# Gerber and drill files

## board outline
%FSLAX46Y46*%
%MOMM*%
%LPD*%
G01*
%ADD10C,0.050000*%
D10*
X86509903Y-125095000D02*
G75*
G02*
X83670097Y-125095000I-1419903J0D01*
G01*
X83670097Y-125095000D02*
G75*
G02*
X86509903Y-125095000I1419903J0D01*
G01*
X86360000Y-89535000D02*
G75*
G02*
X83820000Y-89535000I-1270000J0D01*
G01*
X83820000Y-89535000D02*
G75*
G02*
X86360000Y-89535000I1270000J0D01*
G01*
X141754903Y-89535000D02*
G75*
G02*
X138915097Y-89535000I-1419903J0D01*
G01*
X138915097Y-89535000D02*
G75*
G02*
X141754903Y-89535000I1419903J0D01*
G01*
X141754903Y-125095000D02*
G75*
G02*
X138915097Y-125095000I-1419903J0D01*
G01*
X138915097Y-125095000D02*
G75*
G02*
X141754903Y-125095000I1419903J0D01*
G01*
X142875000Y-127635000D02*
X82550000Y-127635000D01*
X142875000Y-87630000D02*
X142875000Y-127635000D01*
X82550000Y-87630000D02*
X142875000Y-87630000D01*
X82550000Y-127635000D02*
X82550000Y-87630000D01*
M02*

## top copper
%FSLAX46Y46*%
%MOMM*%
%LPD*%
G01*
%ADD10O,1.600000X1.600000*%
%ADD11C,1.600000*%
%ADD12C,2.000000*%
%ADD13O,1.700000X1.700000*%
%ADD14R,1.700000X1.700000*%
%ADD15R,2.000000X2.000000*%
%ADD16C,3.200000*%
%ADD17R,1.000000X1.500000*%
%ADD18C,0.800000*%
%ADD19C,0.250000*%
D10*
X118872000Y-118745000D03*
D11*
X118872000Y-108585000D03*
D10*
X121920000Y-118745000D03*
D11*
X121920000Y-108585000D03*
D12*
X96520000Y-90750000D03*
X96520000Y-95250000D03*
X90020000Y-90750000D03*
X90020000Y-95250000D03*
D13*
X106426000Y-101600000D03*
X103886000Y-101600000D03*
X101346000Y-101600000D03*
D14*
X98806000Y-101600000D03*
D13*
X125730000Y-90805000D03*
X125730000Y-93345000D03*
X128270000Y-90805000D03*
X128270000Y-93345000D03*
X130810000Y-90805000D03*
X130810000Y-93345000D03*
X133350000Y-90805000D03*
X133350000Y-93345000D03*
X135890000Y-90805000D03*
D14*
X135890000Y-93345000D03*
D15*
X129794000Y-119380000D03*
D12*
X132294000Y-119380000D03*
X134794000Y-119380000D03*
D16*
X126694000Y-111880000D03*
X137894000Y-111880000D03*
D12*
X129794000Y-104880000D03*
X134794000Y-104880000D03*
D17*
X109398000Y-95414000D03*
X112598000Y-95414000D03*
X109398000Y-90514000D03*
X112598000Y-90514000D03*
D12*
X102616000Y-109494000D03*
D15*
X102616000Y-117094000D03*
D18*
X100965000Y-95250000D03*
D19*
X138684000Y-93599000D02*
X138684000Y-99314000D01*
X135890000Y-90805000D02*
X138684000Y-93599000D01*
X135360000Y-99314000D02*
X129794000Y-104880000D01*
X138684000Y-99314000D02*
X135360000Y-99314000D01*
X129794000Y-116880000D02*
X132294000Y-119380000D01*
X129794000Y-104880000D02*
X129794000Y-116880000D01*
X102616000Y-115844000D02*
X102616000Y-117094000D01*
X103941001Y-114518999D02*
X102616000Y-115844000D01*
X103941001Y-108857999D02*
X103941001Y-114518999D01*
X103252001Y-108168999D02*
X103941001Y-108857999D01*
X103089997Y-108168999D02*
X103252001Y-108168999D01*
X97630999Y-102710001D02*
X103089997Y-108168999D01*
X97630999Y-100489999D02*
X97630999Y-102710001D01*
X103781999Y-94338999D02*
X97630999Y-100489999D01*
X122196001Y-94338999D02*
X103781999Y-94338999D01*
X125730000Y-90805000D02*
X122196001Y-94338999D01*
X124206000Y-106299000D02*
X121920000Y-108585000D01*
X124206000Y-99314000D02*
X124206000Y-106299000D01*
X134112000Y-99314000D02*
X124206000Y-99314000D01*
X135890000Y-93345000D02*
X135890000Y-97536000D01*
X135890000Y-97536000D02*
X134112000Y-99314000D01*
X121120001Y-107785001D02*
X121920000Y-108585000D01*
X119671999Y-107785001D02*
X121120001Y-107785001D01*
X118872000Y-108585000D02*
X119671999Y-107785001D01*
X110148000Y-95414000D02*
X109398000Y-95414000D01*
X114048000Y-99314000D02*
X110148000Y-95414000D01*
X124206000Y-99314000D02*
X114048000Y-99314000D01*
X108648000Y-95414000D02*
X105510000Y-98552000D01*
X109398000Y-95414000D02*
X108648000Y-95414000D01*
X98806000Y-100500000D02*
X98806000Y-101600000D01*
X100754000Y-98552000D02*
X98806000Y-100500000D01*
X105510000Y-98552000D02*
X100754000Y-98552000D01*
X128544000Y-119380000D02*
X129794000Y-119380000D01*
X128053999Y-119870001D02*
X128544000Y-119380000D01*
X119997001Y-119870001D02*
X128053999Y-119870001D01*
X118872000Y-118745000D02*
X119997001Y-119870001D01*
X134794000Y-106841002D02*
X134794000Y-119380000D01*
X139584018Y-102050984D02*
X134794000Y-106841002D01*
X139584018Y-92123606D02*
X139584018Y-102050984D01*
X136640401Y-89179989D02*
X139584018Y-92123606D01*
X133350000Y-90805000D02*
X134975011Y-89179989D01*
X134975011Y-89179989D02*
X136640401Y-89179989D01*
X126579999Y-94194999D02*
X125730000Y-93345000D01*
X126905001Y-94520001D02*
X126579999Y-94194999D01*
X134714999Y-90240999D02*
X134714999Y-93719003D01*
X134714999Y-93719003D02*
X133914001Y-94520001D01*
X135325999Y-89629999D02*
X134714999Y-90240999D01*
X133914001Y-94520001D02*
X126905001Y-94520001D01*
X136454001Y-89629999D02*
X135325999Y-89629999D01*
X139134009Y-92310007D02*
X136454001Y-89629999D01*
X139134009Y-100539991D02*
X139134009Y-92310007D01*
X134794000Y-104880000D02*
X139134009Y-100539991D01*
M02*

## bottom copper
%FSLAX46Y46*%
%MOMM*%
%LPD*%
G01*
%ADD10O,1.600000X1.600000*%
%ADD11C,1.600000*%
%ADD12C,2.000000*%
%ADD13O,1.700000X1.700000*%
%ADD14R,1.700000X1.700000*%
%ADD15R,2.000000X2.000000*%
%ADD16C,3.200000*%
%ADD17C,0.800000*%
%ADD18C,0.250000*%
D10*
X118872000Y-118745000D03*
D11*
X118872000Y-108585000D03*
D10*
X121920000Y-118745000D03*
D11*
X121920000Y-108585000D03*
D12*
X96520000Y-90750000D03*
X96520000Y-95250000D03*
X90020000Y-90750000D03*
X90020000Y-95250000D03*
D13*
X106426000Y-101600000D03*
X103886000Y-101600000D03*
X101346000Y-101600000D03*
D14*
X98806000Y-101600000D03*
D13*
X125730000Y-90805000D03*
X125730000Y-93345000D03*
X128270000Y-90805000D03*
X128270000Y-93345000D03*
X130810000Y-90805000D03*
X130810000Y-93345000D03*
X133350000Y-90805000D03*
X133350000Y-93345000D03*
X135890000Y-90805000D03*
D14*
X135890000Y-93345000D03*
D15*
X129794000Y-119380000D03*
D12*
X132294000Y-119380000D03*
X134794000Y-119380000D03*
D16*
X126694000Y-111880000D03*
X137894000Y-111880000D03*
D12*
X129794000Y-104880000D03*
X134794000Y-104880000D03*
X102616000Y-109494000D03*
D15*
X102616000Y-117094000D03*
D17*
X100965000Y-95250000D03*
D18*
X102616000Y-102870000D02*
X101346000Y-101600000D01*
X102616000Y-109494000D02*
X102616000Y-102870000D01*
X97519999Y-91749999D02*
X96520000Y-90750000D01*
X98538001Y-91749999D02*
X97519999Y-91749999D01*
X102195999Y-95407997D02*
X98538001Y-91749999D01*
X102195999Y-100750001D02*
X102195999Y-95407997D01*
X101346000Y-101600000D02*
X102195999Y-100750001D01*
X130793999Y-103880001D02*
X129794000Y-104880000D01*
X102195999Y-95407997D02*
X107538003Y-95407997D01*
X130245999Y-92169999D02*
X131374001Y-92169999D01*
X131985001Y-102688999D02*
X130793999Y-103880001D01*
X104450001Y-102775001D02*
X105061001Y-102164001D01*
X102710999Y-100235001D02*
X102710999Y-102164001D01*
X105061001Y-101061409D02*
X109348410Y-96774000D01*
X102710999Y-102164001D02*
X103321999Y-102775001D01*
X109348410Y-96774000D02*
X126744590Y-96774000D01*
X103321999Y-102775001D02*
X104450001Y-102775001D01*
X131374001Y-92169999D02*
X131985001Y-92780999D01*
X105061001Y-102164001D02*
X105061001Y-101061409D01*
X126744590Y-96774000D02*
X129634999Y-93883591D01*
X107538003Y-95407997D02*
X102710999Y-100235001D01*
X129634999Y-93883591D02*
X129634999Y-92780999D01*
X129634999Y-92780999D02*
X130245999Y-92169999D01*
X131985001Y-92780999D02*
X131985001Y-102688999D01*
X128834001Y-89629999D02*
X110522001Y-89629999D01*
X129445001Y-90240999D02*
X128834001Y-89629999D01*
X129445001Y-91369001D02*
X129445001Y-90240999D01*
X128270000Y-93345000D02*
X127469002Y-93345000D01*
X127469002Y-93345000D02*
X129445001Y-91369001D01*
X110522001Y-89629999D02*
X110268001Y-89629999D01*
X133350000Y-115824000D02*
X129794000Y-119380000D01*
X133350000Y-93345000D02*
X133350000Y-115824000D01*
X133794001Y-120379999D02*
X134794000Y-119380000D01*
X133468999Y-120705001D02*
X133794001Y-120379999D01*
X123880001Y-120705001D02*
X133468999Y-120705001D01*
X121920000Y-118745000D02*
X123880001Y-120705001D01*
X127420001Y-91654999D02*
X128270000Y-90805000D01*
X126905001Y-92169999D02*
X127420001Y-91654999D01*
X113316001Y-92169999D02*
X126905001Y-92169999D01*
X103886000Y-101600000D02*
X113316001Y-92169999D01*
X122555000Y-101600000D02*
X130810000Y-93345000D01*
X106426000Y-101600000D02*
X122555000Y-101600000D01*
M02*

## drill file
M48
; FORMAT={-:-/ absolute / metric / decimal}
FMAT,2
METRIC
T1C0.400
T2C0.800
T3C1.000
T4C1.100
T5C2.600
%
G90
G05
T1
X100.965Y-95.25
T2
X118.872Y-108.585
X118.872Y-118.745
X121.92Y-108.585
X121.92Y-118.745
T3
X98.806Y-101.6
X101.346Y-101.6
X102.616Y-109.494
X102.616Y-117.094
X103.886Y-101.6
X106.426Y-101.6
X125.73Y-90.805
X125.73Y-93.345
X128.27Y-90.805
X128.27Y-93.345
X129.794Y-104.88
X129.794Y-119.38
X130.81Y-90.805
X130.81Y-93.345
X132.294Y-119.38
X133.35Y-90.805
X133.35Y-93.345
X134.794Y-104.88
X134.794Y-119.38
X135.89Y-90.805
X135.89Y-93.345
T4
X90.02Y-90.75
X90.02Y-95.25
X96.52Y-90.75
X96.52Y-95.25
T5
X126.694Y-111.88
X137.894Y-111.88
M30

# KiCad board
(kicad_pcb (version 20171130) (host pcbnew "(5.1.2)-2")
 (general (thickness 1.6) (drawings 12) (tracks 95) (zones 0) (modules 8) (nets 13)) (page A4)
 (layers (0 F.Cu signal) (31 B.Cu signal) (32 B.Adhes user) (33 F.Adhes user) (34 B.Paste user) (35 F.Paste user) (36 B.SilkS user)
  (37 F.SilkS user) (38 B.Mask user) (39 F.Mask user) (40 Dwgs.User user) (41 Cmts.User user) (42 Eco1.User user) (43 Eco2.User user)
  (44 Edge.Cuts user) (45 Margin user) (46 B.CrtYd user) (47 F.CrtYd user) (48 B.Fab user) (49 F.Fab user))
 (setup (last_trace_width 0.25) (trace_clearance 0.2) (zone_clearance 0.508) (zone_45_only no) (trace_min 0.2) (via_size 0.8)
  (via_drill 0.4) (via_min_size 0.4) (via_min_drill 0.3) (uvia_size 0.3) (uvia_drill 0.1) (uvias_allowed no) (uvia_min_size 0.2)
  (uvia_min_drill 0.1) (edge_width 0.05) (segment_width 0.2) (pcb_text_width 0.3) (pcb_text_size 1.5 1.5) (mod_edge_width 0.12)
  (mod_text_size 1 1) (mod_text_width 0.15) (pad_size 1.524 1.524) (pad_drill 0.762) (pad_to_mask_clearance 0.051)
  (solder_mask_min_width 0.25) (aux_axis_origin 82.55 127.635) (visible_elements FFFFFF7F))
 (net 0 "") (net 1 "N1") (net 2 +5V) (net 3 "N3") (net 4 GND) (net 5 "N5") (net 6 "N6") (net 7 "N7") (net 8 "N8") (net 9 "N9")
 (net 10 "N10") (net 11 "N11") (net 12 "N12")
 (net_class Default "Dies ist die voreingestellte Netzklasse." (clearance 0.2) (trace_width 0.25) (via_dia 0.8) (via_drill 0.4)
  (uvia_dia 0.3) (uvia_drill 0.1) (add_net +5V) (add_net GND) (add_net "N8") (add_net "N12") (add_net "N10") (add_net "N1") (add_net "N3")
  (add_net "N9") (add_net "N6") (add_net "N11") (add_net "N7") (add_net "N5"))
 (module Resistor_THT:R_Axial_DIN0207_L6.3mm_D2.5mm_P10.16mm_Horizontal (layer F.Cu) (at 118.872 108.585 270)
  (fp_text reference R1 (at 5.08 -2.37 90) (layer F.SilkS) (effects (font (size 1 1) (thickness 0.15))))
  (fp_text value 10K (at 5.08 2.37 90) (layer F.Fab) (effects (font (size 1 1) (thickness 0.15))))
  (pad 2 thru_hole oval (at 10.16 0 270) (size 1.6 1.6) (drill 0.8) (layers *.Cu *.Mask) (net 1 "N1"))
  (pad 1 thru_hole circle (at 0 0 270) (size 1.6 1.6) (drill 0.8) (layers *.Cu *.Mask) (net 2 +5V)))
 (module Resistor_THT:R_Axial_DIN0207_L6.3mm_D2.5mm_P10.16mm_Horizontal (layer F.Cu) (at 121.92 108.585 270)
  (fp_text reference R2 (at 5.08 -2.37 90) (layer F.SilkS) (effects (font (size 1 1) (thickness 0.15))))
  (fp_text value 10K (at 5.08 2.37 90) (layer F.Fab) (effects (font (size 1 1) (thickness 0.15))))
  (pad 2 thru_hole oval (at 10.16 0 270) (size 1.6 1.6) (drill 0.8) (layers *.Cu *.Mask) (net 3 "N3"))
  (pad 1 thru_hole circle (at 0 0 270) (size 1.6 1.6) (drill 0.8) (layers *.Cu *.Mask) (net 2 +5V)))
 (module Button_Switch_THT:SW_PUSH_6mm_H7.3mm (layer F.Cu) (at 90.02 90.75)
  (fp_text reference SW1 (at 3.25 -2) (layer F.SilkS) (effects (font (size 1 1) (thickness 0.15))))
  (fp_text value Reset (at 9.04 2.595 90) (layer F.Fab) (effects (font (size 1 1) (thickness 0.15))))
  (pad 1 thru_hole circle (at 6.5 0 90) (size 2 2) (drill 1.1) (layers *.Cu *.Mask) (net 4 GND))
  (pad 2 thru_hole circle (at 6.5 4.5 90) (size 2 2) (drill 1.1) (layers *.Cu *.Mask) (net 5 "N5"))
  (pad 1 thru_hole circle (at 0 0 90) (size 2 2) (drill 1.1) (layers *.Cu *.Mask) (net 4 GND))
  (pad 2 thru_hole circle (at 0 4.5 90) (size 2 2) (drill 1.1) (layers *.Cu *.Mask) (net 5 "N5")))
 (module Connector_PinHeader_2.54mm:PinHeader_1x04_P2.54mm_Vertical (layer F.Cu) (at 98.806 101.6 90)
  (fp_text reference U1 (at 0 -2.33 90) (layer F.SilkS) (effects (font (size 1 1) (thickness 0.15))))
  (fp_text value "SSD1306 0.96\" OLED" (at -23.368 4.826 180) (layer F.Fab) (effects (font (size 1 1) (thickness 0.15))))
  (pad 4 thru_hole oval (at 0 7.62 90) (size 1.7 1.7) (drill 1) (layers *.Cu *.Mask) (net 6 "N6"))
  (pad 3 thru_hole oval (at 0 5.08 90) (size 1.7 1.7) (drill 1) (layers *.Cu *.Mask) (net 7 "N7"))
  (pad 2 thru_hole oval (at 0 2.54 90) (size 1.7 1.7) (drill 1) (layers *.Cu *.Mask) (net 4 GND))
  (pad 1 thru_hole rect (at 0 0 90) (size 1.7 1.7) (drill 1) (layers *.Cu *.Mask) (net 2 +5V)))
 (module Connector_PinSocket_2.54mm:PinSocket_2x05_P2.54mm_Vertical (layer F.Cu) (at 135.89 93.345 270)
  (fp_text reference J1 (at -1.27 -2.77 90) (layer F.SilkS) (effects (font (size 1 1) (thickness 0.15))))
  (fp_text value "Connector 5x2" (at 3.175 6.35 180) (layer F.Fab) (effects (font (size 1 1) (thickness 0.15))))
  (pad 10 thru_hole oval (at -2.54 10.16 270) (size 1.7 1.7) (drill 1) (layers *.Cu *.Mask) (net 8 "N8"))
  (pad 9 thru_hole oval (at 0 10.16 270) (size 1.7 1.7) (drill 1) (layers *.Cu *.Mask) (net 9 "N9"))
  (pad 8 thru_hole oval (at -2.54 7.62 270) (size 1.7 1.7) (drill 1) (layers *.Cu *.Mask) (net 7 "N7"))
  (pad 7 thru_hole oval (at 0 7.62 270) (size 1.7 1.7) (drill 1) (layers *.Cu *.Mask) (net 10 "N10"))
  (pad 6 thru_hole oval (at -2.54 5.08 270) (size 1.7 1.7) (drill 1) (layers *.Cu *.Mask) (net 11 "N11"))
  (pad 5 thru_hole oval (at 0 5.08 270) (size 1.7 1.7) (drill 1) (layers *.Cu *.Mask) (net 6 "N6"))
  (pad 4 thru_hole oval (at -2.54 2.54 270) (size 1.7 1.7) (drill 1) (layers *.Cu *.Mask) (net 3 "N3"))
  (pad 3 thru_hole oval (at 0 2.54 270) (size 1.7 1.7) (drill 1) (layers *.Cu *.Mask) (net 1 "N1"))
  (pad 2 thru_hole oval (at -2.54 0 270) (size 1.7 1.7) (drill 1) (layers *.Cu *.Mask) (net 4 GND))
  (pad 1 thru_hole rect (at 0 0 270) (size 1.7 1.7) (drill 1) (layers *.Cu *.Mask) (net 2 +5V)))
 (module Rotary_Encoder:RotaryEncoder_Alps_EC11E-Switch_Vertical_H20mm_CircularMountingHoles (layer F.Cu) (at 129.794 119.38 90)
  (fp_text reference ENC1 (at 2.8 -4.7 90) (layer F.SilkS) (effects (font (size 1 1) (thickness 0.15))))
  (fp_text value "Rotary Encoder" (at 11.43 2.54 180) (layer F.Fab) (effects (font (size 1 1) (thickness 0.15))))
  (pad A thru_hole rect (at 0 0 90) (size 2 2) (drill 1) (layers *.Cu *.Mask) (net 1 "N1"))
  (pad C thru_hole circle (at 0 2.5 90) (size 2 2) (drill 1) (layers *.Cu *.Mask) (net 4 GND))
  (pad B thru_hole circle (at 0 5 90) (size 2 2) (drill 1) (layers *.Cu *.Mask) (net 3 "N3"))
  (pad MP thru_hole circle (at 7.5 -3.1 90) (size 3.2 3.2) (drill 2.6) (layers *.Cu *.Mask))
  (pad MP thru_hole circle (at 7.5 8.1 90) (size 3.2 3.2) (drill 2.6) (layers *.Cu *.Mask))
  (pad S2 thru_hole circle (at 14.5 0 90) (size 2 2) (drill 1) (layers *.Cu *.Mask) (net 4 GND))
  (pad S1 thru_hole circle (at 14.5 5 90) (size 2 2) (drill 1) (layers *.Cu *.Mask) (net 9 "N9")))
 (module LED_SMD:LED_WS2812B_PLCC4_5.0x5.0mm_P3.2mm (layer F.Cu) (at 110.998 92.964 90)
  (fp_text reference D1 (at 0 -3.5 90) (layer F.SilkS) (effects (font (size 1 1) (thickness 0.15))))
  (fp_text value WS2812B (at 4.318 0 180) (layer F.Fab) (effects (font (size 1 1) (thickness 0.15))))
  (pad 1 smd rect (at -2.45 -1.6 90) (size 1.5 1) (layers F.Cu F.Paste F.Mask) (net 2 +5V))
  (pad 2 smd rect (at -2.45 1.6 90) (size 1.5 1) (layers F.Cu F.Paste F.Mask) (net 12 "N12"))
  (pad 4 smd rect (at 2.45 -1.6 90) (size 1.5 1) (layers F.Cu F.Paste F.Mask) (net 10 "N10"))
  (pad 3 smd rect (at 2.45 1.6 90) (size 1.5 1) (layers F.Cu F.Paste F.Mask) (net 4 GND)))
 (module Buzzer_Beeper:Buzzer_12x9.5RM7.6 (layer F.Cu) (at 102.616 117.094 90)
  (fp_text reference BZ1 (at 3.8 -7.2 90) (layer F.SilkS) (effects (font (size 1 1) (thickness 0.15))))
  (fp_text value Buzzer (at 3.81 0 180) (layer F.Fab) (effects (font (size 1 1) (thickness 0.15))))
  (pad 2 thru_hole circle (at 7.6 0 90) (size 2 2) (drill 1) (layers *.Cu *.Mask) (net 4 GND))
  (pad 1 thru_hole rect (at 0 0 90) (size 2 2) (drill 1) (layers *.Cu *.Mask) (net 8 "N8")))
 (gr_circle (center 85.09 125.095) (end 85.725 126.365) (layer Edge.Cuts) (width 0.05))
 (gr_circle (center 85.09 89.535) (end 85.09 90.805) (layer Edge.Cuts) (width 0.05))
 (gr_circle (center 140.335 89.535) (end 140.97 90.805) (layer Edge.Cuts) (width 0.05))
 (gr_circle (center 140.335 125.095) (end 139.7 126.365) (layer Edge.Cuts) (width 0.05))
 (gr_line (start 142.875 127.635) (end 82.55 127.635) (layer Edge.Cuts) (width 0.05))
 (gr_line (start 142.875 87.63) (end 142.875 127.635) (layer Edge.Cuts) (width 0.05))
 (gr_line (start 82.55 87.63) (end 142.875 87.63) (layer Edge.Cuts) (width 0.05))
 (gr_line (start 82.55 127.635) (end 82.55 87.63) (layer Edge.Cuts) (width 0.05))
 (via (at 100.965 95.25) (size 0.8) (drill 0.4) (layers F.Cu B.Cu) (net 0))
 (segment (start 138.684 93.599) (end 138.684 99.314) (width 0.25) (layer F.Cu) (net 4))
 (segment (start 135.89 90.805) (end 138.684 93.599) (width 0.25) (layer F.Cu) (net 4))
 (segment (start 135.36 99.314) (end 129.794 104.88) (width 0.25) (layer F.Cu) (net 4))
 (segment (start 138.684 99.314) (end 135.36 99.314) (width 0.25) (layer F.Cu) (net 4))
 (segment (start 129.794 116.88) (end 132.294 119.38) (width 0.25) (layer F.Cu) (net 4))
 (segment (start 129.794 104.88) (end 129.794 116.88) (width 0.25) (layer F.Cu) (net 4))
 (segment (start 102.616 102.87) (end 101.346 101.6) (width 0.25) (layer B.Cu) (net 4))
 (segment (start 102.616 109.494) (end 102.616 102.87) (width 0.25) (layer B.Cu) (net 4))
 (segment (start 97.519999 91.749999) (end 96.52 90.75) (width 0.25) (layer B.Cu) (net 4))
 (segment (start 98.538001 91.749999) (end 97.519999 91.749999) (width 0.25) (layer B.Cu) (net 4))
 (segment (start 102.195999 95.407997) (end 98.538001 91.749999) (width 0.25) (layer B.Cu) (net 4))
 (segment (start 102.195999 100.750001) (end 102.195999 95.407997) (width 0.25) (layer B.Cu) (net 4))
 (segment (start 101.346 101.6) (end 102.195999 100.750001) (width 0.25) (layer B.Cu) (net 4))
 (segment (start 130.793999 103.880001) (end 129.794 104.88) (width 0.25) (layer B.Cu) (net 4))
 (segment (start 102.195999 95.407997) (end 107.538003 95.407997) (width 0.25) (layer B.Cu) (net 4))
 (segment (start 130.245999 92.169999) (end 131.374001 92.169999) (width 0.25) (layer B.Cu) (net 4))
 (segment (start 131.985001 102.688999) (end 130.793999 103.880001) (width 0.25) (layer B.Cu) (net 4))
 (segment (start 104.450001 102.775001) (end 105.061001 102.164001) (width 0.25) (layer B.Cu) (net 4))
 (segment (start 102.710999 100.235001) (end 102.710999 102.164001) (width 0.25) (layer B.Cu) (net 4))
 (segment (start 105.061001 101.061409) (end 109.34841 96.774) (width 0.25) (layer B.Cu) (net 4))
 (segment (start 102.710999 102.164001) (end 103.321999 102.775001) (width 0.25) (layer B.Cu) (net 4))
 (segment (start 109.34841 96.774) (end 126.74459 96.774) (width 0.25) (layer B.Cu) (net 4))
 (segment (start 103.321999 102.775001) (end 104.450001 102.775001) (width 0.25) (layer B.Cu) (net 4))
 (segment (start 131.374001 92.169999) (end 131.985001 92.780999) (width 0.25) (layer B.Cu) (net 4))
 (segment (start 105.061001 102.164001) (end 105.061001 101.061409) (width 0.25) (layer B.Cu) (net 4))
 (segment (start 126.74459 96.774) (end 129.634999 93.883591) (width 0.25) (layer B.Cu) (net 4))
 (segment (start 107.538003 95.407997) (end 102.710999 100.235001) (width 0.25) (layer B.Cu) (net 4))
 (segment (start 129.634999 93.883591) (end 129.634999 92.780999) (width 0.25) (layer B.Cu) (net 4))
 (segment (start 129.634999 92.780999) (end 130.245999 92.169999) (width 0.25) (layer B.Cu) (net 4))
 (segment (start 131.985001 92.780999) (end 131.985001 102.688999) (width 0.25) (layer B.Cu) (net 4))
 (segment (start 102.616 115.844) (end 102.616 117.094) (width 0.25) (layer F.Cu) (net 8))
 (segment (start 103.941001 114.518999) (end 102.616 115.844) (width 0.25) (layer F.Cu) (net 8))
 (segment (start 103.941001 108.857999) (end 103.941001 114.518999) (width 0.25) (layer F.Cu) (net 8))
 (segment (start 103.252001 108.168999) (end 103.941001 108.857999) (width 0.25) (layer F.Cu) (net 8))
 (segment (start 103.089997 108.168999) (end 103.252001 108.168999) (width 0.25) (layer F.Cu) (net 8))
 (segment (start 97.630999 102.710001) (end 103.089997 108.168999) (width 0.25) (layer F.Cu) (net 8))
 (segment (start 97.630999 100.489999) (end 97.630999 102.710001) (width 0.25) (layer F.Cu) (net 8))
 (segment (start 103.781999 94.338999) (end 97.630999 100.489999) (width 0.25) (layer F.Cu) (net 8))
 (segment (start 122.196001 94.338999) (end 103.781999 94.338999) (width 0.25) (layer F.Cu) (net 8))
 (segment (start 125.73 90.805) (end 122.196001 94.338999) (width 0.25) (layer F.Cu) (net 8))
 (segment (start 124.206 106.299) (end 121.92 108.585) (width 0.25) (layer F.Cu) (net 2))
 (segment (start 124.206 99.314) (end 124.206 106.299) (width 0.25) (layer F.Cu) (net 2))
 (segment (start 134.112 99.314) (end 124.206 99.314) (width 0.25) (layer F.Cu) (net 2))
 (segment (start 135.89 93.345) (end 135.89 97.536) (width 0.25) (layer F.Cu) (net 2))
 (segment (start 135.89 97.536) (end 134.112 99.314) (width 0.25) (layer F.Cu) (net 2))
 (segment (start 121.120001 107.785001) (end 121.92 108.585) (width 0.25) (layer F.Cu) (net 2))
 (segment (start 119.671999 107.785001) (end 121.120001 107.785001) (width 0.25) (layer F.Cu) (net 2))
 (segment (start 118.872 108.585) (end 119.671999 107.785001) (width 0.25) (layer F.Cu) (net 2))
 (segment (start 110.148 95.414) (end 109.398 95.414) (width 0.25) (layer F.Cu) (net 2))
 (segment (start 114.048 99.314) (end 110.148 95.414) (width 0.25) (layer F.Cu) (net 2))
 (segment (start 124.206 99.314) (end 114.048 99.314) (width 0.25) (layer F.Cu) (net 2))
 (segment (start 108.648 95.414) (end 105.51 98.552) (width 0.25) (layer F.Cu) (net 2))
 (segment (start 109.398 95.414) (end 108.648 95.414) (width 0.25) (layer F.Cu) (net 2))
 (segment (start 98.806 100.5) (end 98.806 101.6) (width 0.25) (layer F.Cu) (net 2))
 (segment (start 100.754 98.552) (end 98.806 100.5) (width 0.25) (layer F.Cu) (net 2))
 (segment (start 105.51 98.552) (end 100.754 98.552) (width 0.25) (layer F.Cu) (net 2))
 (segment (start 128.834001 89.629999) (end 110.522001 89.629999) (width 0.25) (layer B.Cu) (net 10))
 (segment (start 129.445001 90.240999) (end 128.834001 89.629999) (width 0.25) (layer B.Cu) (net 10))
 (segment (start 129.445001 91.369001) (end 129.445001 90.240999) (width 0.25) (layer B.Cu) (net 10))
 (segment (start 128.27 93.345) (end 127.469002 93.345) (width 0.25) (layer B.Cu) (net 10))
 (segment (start 127.469002 93.345) (end 129.445001 91.369001) (width 0.25) (layer B.Cu) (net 10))
 (segment (start 110.522001 89.629999) (end 110.268001 89.629999) (width 0.25) (layer B.Cu) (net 10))
 (segment (start 128.544 119.38) (end 129.794 119.38) (width 0.25) (layer F.Cu) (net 1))
 (segment (start 128.053999 119.870001) (end 128.544 119.38) (width 0.25) (layer F.Cu) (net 1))
 (segment (start 119.997001 119.870001) (end 128.053999 119.870001) (width 0.25) (layer F.Cu) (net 1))
 (segment (start 118.872 118.745) (end 119.997001 119.870001) (width 0.25) (layer F.Cu) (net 1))
 (segment (start 133.35 115.824) (end 129.794 119.38) (width 0.25) (layer B.Cu) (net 1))
 (segment (start 133.35 93.345) (end 133.35 115.824) (width 0.25) (layer B.Cu) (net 1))
 (segment (start 134.794 106.841002) (end 134.794 119.38) (width 0.25) (layer F.Cu) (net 3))
 (segment (start 139.584018 102.050984) (end 134.794 106.841002) (width 0.25) (layer F.Cu) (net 3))
 (segment (start 139.584018 92.123606) (end 139.584018 102.050984) (width 0.25) (layer F.Cu) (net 3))
 (segment (start 136.640401 89.179989) (end 139.584018 92.123606) (width 0.25) (layer F.Cu) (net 3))
 (segment (start 133.35 90.805) (end 134.975011 89.179989) (width 0.25) (layer F.Cu) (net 3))
 (segment (start 134.975011 89.179989) (end 136.640401 89.179989) (width 0.25) (layer F.Cu) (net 3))
 (segment (start 133.794001 120.379999) (end 134.794 119.38) (width 0.25) (layer B.Cu) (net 3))
 (segment (start 133.468999 120.705001) (end 133.794001 120.379999) (width 0.25) (layer B.Cu) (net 3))
 (segment (start 123.880001 120.705001) (end 133.468999 120.705001) (width 0.25) (layer B.Cu) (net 3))
 (segment (start 121.92 118.745) (end 123.880001 120.705001) (width 0.25) (layer B.Cu) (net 3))
 (segment (start 126.579999 94.194999) (end 125.73 93.345) (width 0.25) (layer F.Cu) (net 9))
 (segment (start 126.905001 94.520001) (end 126.579999 94.194999) (width 0.25) (layer F.Cu) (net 9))
 (segment (start 134.714999 90.240999) (end 134.714999 93.719003) (width 0.25) (layer F.Cu) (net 9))
 (segment (start 134.714999 93.719003) (end 133.914001 94.520001) (width 0.25) (layer F.Cu) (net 9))
 (segment (start 135.325999 89.629999) (end 134.714999 90.240999) (width 0.25) (layer F.Cu) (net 9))
 (segment (start 133.914001 94.520001) (end 126.905001 94.520001) (width 0.25) (layer F.Cu) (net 9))
 (segment (start 136.454001 89.629999) (end 135.325999 89.629999) (width 0.25) (layer F.Cu) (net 9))
 (segment (start 139.134009 92.310007) (end 136.454001 89.629999) (width 0.25) (layer F.Cu) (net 9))
 (segment (start 139.134009 100.539991) (end 139.134009 92.310007) (width 0.25) (layer F.Cu) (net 9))
 (segment (start 134.794 104.88) (end 139.134009 100.539991) (width 0.25) (layer F.Cu) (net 9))
 (segment (start 127.420001 91.654999) (end 128.27 90.805) (width 0.25) (layer B.Cu) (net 7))
 (segment (start 126.905001 92.169999) (end 127.420001 91.654999) (width 0.25) (layer B.Cu) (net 7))
 (segment (start 113.316001 92.169999) (end 126.905001 92.169999) (width 0.25) (layer B.Cu) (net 7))
 (segment (start 103.886 101.6) (end 113.316001 92.169999) (width 0.25) (layer B.Cu) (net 7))
 (segment (start 122.555 101.6) (end 130.81 93.345) (width 0.25) (layer B.Cu) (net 6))
 (segment (start 106.426 101.6) (end 122.555 101.6) (width 0.25) (layer B.Cu) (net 6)))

